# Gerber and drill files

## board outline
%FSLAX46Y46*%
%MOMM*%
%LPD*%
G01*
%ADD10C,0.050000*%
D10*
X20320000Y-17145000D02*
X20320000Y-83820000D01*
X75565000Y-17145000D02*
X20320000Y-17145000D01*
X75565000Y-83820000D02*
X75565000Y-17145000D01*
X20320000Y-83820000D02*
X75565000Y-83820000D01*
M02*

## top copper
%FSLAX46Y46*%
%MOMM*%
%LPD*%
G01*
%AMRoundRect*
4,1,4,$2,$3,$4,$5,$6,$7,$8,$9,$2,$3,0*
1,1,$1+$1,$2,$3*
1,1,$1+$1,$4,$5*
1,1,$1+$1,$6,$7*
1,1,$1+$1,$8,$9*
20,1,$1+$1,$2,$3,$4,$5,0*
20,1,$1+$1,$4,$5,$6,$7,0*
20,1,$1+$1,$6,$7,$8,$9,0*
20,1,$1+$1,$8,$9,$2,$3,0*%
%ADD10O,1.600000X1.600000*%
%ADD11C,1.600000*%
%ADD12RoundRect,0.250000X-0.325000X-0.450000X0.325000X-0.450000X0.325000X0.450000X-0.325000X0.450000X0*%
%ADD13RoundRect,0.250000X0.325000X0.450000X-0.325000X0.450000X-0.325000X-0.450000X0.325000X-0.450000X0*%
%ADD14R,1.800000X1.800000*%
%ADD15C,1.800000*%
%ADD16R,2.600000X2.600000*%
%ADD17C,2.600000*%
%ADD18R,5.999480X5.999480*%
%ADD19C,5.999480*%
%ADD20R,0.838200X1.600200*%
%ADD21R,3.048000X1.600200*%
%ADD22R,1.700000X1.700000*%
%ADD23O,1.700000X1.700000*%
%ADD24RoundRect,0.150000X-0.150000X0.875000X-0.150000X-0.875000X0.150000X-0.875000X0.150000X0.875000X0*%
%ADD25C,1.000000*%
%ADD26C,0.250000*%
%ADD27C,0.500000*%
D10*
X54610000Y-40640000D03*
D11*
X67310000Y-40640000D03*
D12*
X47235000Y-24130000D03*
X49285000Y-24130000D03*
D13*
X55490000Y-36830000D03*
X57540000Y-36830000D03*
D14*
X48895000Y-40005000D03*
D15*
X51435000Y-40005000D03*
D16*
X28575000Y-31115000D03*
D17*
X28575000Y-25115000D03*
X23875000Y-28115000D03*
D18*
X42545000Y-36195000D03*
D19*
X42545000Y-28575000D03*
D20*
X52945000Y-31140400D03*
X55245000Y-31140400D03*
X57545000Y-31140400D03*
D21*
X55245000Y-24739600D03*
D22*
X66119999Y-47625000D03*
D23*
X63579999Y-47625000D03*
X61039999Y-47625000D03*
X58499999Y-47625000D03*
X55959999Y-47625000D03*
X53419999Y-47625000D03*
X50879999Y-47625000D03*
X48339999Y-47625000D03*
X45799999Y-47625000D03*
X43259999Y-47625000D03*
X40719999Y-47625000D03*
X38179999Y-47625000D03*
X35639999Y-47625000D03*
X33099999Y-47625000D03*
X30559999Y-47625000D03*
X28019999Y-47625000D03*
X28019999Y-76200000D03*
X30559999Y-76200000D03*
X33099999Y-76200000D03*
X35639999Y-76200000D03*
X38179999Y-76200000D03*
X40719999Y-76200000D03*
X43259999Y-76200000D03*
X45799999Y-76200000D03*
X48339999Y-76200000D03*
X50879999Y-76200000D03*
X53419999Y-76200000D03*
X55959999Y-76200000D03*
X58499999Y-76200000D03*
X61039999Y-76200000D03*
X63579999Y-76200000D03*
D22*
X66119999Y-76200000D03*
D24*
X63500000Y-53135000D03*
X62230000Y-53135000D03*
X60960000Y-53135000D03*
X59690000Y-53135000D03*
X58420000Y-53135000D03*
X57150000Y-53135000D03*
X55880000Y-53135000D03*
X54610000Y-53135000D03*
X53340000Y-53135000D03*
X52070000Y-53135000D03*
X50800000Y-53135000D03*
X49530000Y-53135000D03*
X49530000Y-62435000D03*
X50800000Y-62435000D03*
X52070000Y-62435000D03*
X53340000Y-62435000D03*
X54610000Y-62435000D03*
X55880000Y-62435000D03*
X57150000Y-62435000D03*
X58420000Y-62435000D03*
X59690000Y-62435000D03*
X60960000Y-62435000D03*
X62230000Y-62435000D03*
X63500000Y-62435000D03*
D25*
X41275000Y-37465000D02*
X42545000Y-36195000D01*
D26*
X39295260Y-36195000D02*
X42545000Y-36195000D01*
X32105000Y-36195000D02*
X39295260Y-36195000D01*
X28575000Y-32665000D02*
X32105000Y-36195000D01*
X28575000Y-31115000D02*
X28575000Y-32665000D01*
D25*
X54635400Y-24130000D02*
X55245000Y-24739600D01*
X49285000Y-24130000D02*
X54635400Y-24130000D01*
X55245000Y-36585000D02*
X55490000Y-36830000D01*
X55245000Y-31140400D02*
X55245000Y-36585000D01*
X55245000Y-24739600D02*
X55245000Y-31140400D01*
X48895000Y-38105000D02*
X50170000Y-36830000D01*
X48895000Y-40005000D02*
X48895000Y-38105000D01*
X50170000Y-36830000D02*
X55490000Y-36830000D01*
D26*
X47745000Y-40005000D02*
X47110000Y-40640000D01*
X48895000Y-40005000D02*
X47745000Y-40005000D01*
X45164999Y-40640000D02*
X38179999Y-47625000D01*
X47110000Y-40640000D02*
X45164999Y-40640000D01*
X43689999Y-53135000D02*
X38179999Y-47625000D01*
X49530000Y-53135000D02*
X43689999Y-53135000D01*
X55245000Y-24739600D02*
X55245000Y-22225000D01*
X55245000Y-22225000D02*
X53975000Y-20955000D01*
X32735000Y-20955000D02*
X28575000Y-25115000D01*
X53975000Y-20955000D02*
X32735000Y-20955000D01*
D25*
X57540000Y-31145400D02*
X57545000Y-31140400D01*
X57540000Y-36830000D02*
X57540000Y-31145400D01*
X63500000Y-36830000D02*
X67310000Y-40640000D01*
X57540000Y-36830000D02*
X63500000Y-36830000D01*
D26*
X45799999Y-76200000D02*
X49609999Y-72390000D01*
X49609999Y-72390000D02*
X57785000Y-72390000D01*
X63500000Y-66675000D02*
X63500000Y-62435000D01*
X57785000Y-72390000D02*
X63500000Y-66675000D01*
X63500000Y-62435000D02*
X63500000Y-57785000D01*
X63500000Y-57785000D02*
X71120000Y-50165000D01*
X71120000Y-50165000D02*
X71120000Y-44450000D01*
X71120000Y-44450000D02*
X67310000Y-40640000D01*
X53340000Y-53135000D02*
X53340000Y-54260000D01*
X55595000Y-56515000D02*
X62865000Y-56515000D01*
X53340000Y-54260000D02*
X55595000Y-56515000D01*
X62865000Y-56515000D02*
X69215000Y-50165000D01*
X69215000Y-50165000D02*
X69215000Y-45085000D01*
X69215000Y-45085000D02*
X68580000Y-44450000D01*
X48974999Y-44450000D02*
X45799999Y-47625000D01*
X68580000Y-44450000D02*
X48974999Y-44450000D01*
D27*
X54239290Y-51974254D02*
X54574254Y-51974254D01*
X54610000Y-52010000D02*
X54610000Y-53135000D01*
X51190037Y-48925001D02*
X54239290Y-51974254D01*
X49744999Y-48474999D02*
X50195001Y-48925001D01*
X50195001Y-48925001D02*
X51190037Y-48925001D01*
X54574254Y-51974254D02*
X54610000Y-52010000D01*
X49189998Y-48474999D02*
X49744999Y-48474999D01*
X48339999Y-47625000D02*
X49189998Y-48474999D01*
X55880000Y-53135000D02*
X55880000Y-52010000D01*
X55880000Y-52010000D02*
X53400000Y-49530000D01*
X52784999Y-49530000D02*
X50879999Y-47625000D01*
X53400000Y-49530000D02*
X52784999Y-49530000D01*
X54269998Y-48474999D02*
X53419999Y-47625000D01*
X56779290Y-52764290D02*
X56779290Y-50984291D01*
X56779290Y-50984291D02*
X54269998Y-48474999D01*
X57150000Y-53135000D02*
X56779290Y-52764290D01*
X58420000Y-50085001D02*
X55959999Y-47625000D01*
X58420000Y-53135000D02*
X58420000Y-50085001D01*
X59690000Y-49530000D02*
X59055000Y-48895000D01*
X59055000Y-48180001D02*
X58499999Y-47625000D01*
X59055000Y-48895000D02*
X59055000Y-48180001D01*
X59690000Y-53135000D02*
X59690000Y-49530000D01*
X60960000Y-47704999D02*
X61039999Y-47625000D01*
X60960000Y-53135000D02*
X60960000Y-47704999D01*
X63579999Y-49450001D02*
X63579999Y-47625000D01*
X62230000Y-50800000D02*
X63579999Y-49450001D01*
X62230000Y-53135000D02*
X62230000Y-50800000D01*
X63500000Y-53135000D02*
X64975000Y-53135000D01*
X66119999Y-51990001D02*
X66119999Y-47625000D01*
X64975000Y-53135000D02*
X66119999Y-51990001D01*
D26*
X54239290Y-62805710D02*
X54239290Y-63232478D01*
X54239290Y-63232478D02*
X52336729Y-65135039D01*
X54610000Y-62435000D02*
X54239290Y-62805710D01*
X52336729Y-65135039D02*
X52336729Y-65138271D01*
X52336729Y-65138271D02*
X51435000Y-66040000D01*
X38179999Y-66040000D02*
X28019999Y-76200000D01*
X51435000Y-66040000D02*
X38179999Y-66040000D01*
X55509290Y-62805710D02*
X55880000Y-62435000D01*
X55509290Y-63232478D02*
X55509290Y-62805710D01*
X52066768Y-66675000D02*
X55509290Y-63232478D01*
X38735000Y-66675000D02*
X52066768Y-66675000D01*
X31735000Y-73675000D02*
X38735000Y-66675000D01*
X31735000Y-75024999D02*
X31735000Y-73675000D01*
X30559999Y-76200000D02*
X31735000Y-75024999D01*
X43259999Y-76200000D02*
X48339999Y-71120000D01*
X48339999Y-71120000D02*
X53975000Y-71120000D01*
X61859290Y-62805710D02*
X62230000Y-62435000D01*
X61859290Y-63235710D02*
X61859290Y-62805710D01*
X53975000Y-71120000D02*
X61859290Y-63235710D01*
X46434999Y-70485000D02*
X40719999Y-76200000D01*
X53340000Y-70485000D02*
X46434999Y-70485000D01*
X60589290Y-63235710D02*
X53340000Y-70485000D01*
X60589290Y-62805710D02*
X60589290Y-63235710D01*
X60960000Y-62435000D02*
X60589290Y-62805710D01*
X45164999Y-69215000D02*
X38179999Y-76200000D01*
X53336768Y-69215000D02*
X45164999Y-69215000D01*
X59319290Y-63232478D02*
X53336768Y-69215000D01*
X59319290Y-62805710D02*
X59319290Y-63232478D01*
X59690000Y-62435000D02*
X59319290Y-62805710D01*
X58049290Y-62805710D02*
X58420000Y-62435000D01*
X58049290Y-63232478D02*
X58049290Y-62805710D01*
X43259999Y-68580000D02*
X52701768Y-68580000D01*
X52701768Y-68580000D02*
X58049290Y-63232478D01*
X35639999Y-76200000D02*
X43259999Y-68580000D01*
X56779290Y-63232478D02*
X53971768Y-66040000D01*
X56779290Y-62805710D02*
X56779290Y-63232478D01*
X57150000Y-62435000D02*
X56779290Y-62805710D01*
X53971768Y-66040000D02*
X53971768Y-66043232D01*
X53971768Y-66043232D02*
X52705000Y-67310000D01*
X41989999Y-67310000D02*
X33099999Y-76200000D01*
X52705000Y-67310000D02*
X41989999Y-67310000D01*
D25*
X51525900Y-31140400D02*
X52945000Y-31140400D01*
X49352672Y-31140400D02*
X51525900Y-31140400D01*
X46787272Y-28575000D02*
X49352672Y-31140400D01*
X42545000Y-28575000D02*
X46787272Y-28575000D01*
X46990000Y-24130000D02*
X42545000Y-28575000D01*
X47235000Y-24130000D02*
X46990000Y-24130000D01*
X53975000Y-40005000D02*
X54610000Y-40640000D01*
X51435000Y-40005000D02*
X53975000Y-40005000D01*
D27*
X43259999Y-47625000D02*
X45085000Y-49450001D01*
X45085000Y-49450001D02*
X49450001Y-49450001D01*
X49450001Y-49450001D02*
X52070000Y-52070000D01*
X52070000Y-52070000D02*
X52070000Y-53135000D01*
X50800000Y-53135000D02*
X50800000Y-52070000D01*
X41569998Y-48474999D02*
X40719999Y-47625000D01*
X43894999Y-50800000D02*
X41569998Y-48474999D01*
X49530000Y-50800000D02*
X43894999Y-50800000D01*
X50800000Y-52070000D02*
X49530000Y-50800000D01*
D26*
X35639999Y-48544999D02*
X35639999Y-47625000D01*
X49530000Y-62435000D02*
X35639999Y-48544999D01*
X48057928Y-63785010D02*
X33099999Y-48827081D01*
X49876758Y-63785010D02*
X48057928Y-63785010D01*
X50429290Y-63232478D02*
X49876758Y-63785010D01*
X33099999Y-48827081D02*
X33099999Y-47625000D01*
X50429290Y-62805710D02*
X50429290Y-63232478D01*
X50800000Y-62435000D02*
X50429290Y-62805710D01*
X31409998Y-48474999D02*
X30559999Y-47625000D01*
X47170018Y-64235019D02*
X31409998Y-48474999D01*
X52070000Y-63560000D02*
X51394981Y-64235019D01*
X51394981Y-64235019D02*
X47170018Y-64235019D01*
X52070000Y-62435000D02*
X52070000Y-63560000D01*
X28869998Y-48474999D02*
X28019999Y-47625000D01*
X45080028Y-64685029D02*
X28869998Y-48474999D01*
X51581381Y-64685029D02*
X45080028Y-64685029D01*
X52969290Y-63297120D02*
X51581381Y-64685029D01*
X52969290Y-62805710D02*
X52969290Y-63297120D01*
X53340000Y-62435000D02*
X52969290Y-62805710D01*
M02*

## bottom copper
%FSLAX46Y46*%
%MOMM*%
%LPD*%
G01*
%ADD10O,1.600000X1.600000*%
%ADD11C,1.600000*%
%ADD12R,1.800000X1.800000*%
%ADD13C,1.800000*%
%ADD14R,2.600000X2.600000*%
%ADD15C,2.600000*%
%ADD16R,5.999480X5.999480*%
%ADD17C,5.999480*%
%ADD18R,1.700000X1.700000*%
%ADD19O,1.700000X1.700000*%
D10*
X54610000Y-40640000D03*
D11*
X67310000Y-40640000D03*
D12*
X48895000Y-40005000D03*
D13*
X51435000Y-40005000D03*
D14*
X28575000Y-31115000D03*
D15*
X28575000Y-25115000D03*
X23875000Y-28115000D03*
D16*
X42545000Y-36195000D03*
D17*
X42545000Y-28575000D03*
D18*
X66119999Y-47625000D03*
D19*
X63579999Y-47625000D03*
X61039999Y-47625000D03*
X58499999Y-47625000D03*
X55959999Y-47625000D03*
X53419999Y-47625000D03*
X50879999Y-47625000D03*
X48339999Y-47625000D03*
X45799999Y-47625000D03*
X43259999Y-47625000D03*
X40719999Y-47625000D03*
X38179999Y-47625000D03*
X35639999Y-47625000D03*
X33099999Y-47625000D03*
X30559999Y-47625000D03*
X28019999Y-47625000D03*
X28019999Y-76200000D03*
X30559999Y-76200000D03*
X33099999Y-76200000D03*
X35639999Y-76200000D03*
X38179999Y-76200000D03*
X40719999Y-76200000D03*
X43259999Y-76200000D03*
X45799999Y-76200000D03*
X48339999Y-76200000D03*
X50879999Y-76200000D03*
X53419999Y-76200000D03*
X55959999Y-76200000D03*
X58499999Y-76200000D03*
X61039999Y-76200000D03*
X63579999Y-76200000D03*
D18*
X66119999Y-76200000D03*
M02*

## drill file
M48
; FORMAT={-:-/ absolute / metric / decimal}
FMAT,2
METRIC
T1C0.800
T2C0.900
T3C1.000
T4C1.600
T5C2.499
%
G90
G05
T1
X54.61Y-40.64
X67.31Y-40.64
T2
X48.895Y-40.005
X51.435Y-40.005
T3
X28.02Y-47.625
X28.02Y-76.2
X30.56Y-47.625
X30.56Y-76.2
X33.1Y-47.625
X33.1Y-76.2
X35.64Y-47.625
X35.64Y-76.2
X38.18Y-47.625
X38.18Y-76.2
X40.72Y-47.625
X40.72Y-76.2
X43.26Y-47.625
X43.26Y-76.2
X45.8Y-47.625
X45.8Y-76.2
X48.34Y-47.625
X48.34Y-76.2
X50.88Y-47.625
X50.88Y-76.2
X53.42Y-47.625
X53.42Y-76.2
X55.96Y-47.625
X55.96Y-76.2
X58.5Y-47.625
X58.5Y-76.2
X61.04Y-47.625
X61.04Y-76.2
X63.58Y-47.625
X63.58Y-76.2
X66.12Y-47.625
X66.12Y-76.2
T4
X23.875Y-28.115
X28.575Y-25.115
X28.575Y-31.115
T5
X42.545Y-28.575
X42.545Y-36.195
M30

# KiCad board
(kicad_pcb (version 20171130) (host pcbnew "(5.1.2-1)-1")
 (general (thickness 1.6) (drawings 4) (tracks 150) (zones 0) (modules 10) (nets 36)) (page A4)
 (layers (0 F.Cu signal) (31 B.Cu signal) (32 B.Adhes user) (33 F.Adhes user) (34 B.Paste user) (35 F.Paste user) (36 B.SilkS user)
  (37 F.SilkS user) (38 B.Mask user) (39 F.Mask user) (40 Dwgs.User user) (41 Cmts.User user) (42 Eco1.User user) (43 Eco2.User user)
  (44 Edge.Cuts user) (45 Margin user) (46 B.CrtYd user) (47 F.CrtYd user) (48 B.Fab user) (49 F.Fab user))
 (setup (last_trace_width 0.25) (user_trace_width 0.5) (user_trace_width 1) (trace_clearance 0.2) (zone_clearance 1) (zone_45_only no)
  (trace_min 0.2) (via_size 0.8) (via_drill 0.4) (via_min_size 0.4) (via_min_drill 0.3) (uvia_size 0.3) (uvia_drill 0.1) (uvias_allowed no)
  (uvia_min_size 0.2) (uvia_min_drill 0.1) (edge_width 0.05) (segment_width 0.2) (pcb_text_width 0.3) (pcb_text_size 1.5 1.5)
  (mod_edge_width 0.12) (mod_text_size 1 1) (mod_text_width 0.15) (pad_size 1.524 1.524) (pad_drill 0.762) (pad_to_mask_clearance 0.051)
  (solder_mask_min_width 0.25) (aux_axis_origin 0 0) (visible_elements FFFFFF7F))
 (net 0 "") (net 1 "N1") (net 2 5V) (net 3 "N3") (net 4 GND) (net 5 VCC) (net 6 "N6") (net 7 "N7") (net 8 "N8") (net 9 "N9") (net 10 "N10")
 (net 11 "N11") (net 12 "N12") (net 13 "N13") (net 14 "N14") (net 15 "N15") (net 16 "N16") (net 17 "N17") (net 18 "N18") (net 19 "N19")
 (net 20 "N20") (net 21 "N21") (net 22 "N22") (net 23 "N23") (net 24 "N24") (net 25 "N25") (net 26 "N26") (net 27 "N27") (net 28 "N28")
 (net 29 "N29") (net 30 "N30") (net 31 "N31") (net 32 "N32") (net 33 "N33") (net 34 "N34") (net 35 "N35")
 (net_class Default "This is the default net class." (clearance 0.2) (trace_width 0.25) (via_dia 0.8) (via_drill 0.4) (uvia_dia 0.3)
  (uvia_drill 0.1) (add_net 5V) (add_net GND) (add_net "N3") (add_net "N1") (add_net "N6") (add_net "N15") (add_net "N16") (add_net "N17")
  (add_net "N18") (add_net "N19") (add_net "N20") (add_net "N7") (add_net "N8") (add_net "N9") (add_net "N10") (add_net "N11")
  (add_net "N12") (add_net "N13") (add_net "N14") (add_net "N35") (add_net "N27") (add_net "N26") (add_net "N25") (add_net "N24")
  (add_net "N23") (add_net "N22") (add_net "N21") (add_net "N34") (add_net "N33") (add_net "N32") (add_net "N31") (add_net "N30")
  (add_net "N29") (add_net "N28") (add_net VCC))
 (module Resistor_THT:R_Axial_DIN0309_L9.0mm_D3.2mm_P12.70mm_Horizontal (layer F.Cu) (at 67.31 40.64 180)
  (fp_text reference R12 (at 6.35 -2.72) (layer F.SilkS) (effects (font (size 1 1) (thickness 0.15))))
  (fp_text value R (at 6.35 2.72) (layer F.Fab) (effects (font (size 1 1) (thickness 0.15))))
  (pad 2 thru_hole oval (at 12.7 0 180) (size 1.6 1.6) (drill 0.8) (layers *.Cu *.Mask) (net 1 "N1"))
  (pad 1 thru_hole circle (at 0 0 180) (size 1.6 1.6) (drill 0.8) (layers *.Cu *.Mask) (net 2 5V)))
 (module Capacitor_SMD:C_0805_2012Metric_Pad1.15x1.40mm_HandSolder (layer F.Cu) (at 48.26 24.13)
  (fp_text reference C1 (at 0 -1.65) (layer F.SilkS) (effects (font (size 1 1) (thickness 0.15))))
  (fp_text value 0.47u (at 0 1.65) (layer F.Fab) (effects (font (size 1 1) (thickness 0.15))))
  (pad 1 smd roundrect (at -1.025 0) (size 1.15 1.4) (layers F.Cu F.Paste F.Mask) (roundrect_rratio 0.217391) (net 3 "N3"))
  (pad 2 smd roundrect (at 1.025 0) (size 1.15 1.4) (layers F.Cu F.Paste F.Mask) (roundrect_rratio 0.217391) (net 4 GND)))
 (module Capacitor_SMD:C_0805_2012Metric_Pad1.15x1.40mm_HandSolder (layer F.Cu) (at 56.515 36.83 180)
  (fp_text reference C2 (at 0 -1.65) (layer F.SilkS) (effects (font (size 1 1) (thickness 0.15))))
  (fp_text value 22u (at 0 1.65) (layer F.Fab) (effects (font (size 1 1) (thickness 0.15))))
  (pad 2 smd roundrect (at 1.025 0 180) (size 1.15 1.4) (layers F.Cu F.Paste F.Mask) (roundrect_rratio 0.217391) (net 4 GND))
  (pad 1 smd roundrect (at -1.025 0 180) (size 1.15 1.4) (layers F.Cu F.Paste F.Mask) (roundrect_rratio 0.217391) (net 2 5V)))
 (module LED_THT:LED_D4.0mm (layer F.Cu) (at 48.895 40.005)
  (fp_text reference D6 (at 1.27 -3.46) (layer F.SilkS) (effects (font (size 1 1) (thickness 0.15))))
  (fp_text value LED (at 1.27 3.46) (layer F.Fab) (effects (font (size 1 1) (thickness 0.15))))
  (pad 1 thru_hole rect (at 0 0) (size 1.8 1.8) (drill 0.9) (layers *.Cu *.Mask) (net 4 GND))
  (pad 2 thru_hole circle (at 2.54 0) (size 1.8 1.8) (drill 0.9) (layers *.Cu *.Mask) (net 1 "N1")))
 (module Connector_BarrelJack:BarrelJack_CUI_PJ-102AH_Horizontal (layer F.Cu) (at 28.575 31.115 180)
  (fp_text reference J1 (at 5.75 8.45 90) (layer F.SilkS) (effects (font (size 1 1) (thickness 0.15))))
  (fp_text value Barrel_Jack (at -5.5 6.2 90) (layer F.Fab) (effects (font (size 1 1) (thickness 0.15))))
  (pad 1 thru_hole rect (at 0 0 180) (size 2.6 2.6) (drill 1.6) (layers *.Cu *.Mask) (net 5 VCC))
  (pad 2 thru_hole circle (at 0 6 180) (size 2.6 2.6) (drill 1.6) (layers *.Cu *.Mask) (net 4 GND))
  (pad 3 thru_hole circle (at 4.7 3 180) (size 2.6 2.6) (drill 1.6) (layers *.Cu *.Mask)))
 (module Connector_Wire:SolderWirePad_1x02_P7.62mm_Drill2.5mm (layer F.Cu) (at 42.545 36.195 90)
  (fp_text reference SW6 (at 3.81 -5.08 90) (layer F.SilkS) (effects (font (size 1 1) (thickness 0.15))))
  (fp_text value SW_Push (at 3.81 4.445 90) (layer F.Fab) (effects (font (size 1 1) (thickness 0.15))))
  (pad 1 thru_hole rect (at 0 0 90) (size 5.99948 5.99948) (drill 2.49936) (layers *.Cu *.Mask) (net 5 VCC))
  (pad 2 thru_hole circle (at 7.62 0 90) (size 5.99948 5.99948) (drill 2.49936) (layers *.Cu *.Mask) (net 3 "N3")))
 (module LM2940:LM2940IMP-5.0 (layer F.Cu) (at 55.245 27.94 90)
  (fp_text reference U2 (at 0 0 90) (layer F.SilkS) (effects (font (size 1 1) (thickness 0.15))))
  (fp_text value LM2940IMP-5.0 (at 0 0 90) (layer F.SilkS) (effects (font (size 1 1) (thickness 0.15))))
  (pad 1 smd rect (at -3.2004 -2.3 90) (size 1.6002 0.8382) (layers F.Cu F.Paste F.Mask) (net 3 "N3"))
  (pad 2 smd rect (at -3.2004 0 90) (size 1.6002 0.8382) (layers F.Cu F.Paste F.Mask) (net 4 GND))
  (pad 3 smd rect (at -3.2004 2.3 90) (size 1.6002 0.8382) (layers F.Cu F.Paste F.Mask) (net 2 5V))
  (pad 4 smd rect (at 3.2004 0 90) (size 1.6002 3.048) (layers F.Cu F.Paste F.Mask) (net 4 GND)))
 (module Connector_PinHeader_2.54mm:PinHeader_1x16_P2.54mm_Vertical (layer F.Cu) (at 66.119999 47.625 270)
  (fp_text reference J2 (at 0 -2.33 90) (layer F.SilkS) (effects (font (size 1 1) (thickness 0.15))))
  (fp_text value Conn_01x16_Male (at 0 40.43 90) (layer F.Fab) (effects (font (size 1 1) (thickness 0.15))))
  (pad 1 thru_hole rect (at 0 0 270) (size 1.7 1.7) (drill 1) (layers *.Cu *.Mask) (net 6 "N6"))
  (pad 2 thru_hole oval (at 0 2.54 270) (size 1.7 1.7) (drill 1) (layers *.Cu *.Mask) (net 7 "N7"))
  (pad 3 thru_hole oval (at 0 5.08 270) (size 1.7 1.7) (drill 1) (layers *.Cu *.Mask) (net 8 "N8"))
  (pad 4 thru_hole oval (at 0 7.62 270) (size 1.7 1.7) (drill 1) (layers *.Cu *.Mask) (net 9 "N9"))
  (pad 5 thru_hole oval (at 0 10.16 270) (size 1.7 1.7) (drill 1) (layers *.Cu *.Mask) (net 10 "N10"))
  (pad 6 thru_hole oval (at 0 12.7 270) (size 1.7 1.7) (drill 1) (layers *.Cu *.Mask) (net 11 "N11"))
  (pad 7 thru_hole oval (at 0 15.24 270) (size 1.7 1.7) (drill 1) (layers *.Cu *.Mask) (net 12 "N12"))
  (pad 8 thru_hole oval (at 0 17.78 270) (size 1.7 1.7) (drill 1) (layers *.Cu *.Mask) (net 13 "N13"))
  (pad 9 thru_hole oval (at 0 20.32 270) (size 1.7 1.7) (drill 1) (layers *.Cu *.Mask) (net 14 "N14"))
  (pad 10 thru_hole oval (at 0 22.86 270) (size 1.7 1.7) (drill 1) (layers *.Cu *.Mask) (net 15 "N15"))
  (pad 11 thru_hole oval (at 0 25.4 270) (size 1.7 1.7) (drill 1) (layers *.Cu *.Mask) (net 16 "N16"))
  (pad 12 thru_hole oval (at 0 27.94 270) (size 1.7 1.7) (drill 1) (layers *.Cu *.Mask) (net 4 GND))
  (pad 13 thru_hole oval (at 0 30.48 270) (size 1.7 1.7) (drill 1) (layers *.Cu *.Mask) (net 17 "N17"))
  (pad 14 thru_hole oval (at 0 33.02 270) (size 1.7 1.7) (drill 1) (layers *.Cu *.Mask) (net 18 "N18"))
  (pad 15 thru_hole oval (at 0 35.56 270) (size 1.7 1.7) (drill 1) (layers *.Cu *.Mask) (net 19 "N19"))
  (pad 16 thru_hole oval (at 0 38.1 270) (size 1.7 1.7) (drill 1) (layers *.Cu *.Mask) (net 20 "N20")))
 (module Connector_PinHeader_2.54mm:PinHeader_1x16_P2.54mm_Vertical (layer F.Cu) (at 66.119999 76.2 270)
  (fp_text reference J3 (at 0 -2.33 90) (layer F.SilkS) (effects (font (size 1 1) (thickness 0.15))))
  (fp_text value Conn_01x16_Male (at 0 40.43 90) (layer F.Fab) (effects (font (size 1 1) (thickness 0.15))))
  (pad 16 thru_hole oval (at 0 38.1 270) (size 1.7 1.7) (drill 1) (layers *.Cu *.Mask) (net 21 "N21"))
  (pad 15 thru_hole oval (at 0 35.56 270) (size 1.7 1.7) (drill 1) (layers *.Cu *.Mask) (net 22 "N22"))
  (pad 14 thru_hole oval (at 0 33.02 270) (size 1.7 1.7) (drill 1) (layers *.Cu *.Mask) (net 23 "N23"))
  (pad 13 thru_hole oval (at 0 30.48 270) (size 1.7 1.7) (drill 1) (layers *.Cu *.Mask) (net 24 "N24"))
  (pad 12 thru_hole oval (at 0 27.94 270) (size 1.7 1.7) (drill 1) (layers *.Cu *.Mask) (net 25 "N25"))
  (pad 11 thru_hole oval (at 0 25.4 270) (size 1.7 1.7) (drill 1) (layers *.Cu *.Mask) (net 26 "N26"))
  (pad 10 thru_hole oval (at 0 22.86 270) (size 1.7 1.7) (drill 1) (layers *.Cu *.Mask) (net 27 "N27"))
  (pad 9 thru_hole oval (at 0 20.32 270) (size 1.7 1.7) (drill 1) (layers *.Cu *.Mask) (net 2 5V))
  (pad 8 thru_hole oval (at 0 17.78 270) (size 1.7 1.7) (drill 1) (layers *.Cu *.Mask) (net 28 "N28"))
  (pad 7 thru_hole oval (at 0 15.24 270) (size 1.7 1.7) (drill 1) (layers *.Cu *.Mask) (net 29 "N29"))
  (pad 6 thru_hole oval (at 0 12.7 270) (size 1.7 1.7) (drill 1) (layers *.Cu *.Mask) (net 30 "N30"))
  (pad 5 thru_hole oval (at 0 10.16 270) (size 1.7 1.7) (drill 1) (layers *.Cu *.Mask) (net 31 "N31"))
  (pad 4 thru_hole oval (at 0 7.62 270) (size 1.7 1.7) (drill 1) (layers *.Cu *.Mask) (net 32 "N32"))
  (pad 3 thru_hole oval (at 0 5.08 270) (size 1.7 1.7) (drill 1) (layers *.Cu *.Mask) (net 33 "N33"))
  (pad 2 thru_hole oval (at 0 2.54 270) (size 1.7 1.7) (drill 1) (layers *.Cu *.Mask) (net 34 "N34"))
  (pad 1 thru_hole rect (at 0 0 270) (size 1.7 1.7) (drill 1) (layers *.Cu *.Mask) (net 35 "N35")))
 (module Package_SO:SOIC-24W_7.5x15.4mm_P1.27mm (layer F.Cu) (at 56.515 57.785 270)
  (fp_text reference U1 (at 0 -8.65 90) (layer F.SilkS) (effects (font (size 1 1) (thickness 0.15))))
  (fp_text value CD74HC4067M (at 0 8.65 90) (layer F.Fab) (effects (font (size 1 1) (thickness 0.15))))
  (pad 1 smd roundrect (at -4.65 -6.985 270) (size 2.05 0.6) (layers F.Cu F.Paste F.Mask) (roundrect_rratio 0.25) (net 6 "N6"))
  (pad 2 smd roundrect (at -4.65 -5.715 270) (size 2.05 0.6) (layers F.Cu F.Paste F.Mask) (roundrect_rratio 0.25) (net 7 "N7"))
  (pad 3 smd roundrect (at -4.65 -4.445 270) (size 2.05 0.6) (layers F.Cu F.Paste F.Mask) (roundrect_rratio 0.25) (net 8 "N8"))
  (pad 4 smd roundrect (at -4.65 -3.175 270) (size 2.05 0.6) (layers F.Cu F.Paste F.Mask) (roundrect_rratio 0.25) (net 9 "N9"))
  (pad 5 smd roundrect (at -4.65 -1.905 270) (size 2.05 0.6) (layers F.Cu F.Paste F.Mask) (roundrect_rratio 0.25) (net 10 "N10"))
  (pad 6 smd roundrect (at -4.65 -0.635 270) (size 2.05 0.6) (layers F.Cu F.Paste F.Mask) (roundrect_rratio 0.25) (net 11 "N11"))
  (pad 7 smd roundrect (at -4.65 0.635 270) (size 2.05 0.6) (layers F.Cu F.Paste F.Mask) (roundrect_rratio 0.25) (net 12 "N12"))
  (pad 8 smd roundrect (at -4.65 1.905 270) (size 2.05 0.6) (layers F.Cu F.Paste F.Mask) (roundrect_rratio 0.25) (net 13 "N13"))
  (pad 9 smd roundrect (at -4.65 3.175 270) (size 2.05 0.6) (layers F.Cu F.Paste F.Mask) (roundrect_rratio 0.25) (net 14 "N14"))
  (pad 10 smd roundrect (at -4.65 4.445 270) (size 2.05 0.6) (layers F.Cu F.Paste F.Mask) (roundrect_rratio 0.25) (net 15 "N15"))
  (pad 11 smd roundrect (at -4.65 5.715 270) (size 2.05 0.6) (layers F.Cu F.Paste F.Mask) (roundrect_rratio 0.25) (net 16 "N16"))
  (pad 12 smd roundrect (at -4.65 6.985 270) (size 2.05 0.6) (layers F.Cu F.Paste F.Mask) (roundrect_rratio 0.25) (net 4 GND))
  (pad 13 smd roundrect (at 4.65 6.985 270) (size 2.05 0.6) (layers F.Cu F.Paste F.Mask) (roundrect_rratio 0.25) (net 17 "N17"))
  (pad 14 smd roundrect (at 4.65 5.715 270) (size 2.05 0.6) (layers F.Cu F.Paste F.Mask) (roundrect_rratio 0.25) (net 18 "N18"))
  (pad 15 smd roundrect (at 4.65 4.445 270) (size 2.05 0.6) (layers F.Cu F.Paste F.Mask) (roundrect_rratio 0.25) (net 19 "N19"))
  (pad 16 smd roundrect (at 4.65 3.175 270) (size 2.05 0.6) (layers F.Cu F.Paste F.Mask) (roundrect_rratio 0.25) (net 20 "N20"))
  (pad 17 smd roundrect (at 4.65 1.905 270) (size 2.05 0.6) (layers F.Cu F.Paste F.Mask) (roundrect_rratio 0.25) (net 21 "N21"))
  (pad 18 smd roundrect (at 4.65 0.635 270) (size 2.05 0.6) (layers F.Cu F.Paste F.Mask) (roundrect_rratio 0.25) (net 22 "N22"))
  (pad 19 smd roundrect (at 4.65 -0.635 270) (size 2.05 0.6) (layers F.Cu F.Paste F.Mask) (roundrect_rratio 0.25) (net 23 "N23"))
  (pad 20 smd roundrect (at 4.65 -1.905 270) (size 2.05 0.6) (layers F.Cu F.Paste F.Mask) (roundrect_rratio 0.25) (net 24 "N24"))
  (pad 21 smd roundrect (at 4.65 -3.175 270) (size 2.05 0.6) (layers F.Cu F.Paste F.Mask) (roundrect_rratio 0.25) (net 25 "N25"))
  (pad 22 smd roundrect (at 4.65 -4.445 270) (size 2.05 0.6) (layers F.Cu F.Paste F.Mask) (roundrect_rratio 0.25) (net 26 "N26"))
  (pad 23 smd roundrect (at 4.65 -5.715 270) (size 2.05 0.6) (layers F.Cu F.Paste F.Mask) (roundrect_rratio 0.25) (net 27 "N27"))
  (pad 24 smd roundrect (at 4.65 -6.985 270) (size 2.05 0.6) (layers F.Cu F.Paste F.Mask) (roundrect_rratio 0.25) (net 2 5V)))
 (gr_line (start 20.32 17.145) (end 20.32 83.82) (layer Edge.Cuts) (width 0.05))
 (gr_line (start 75.565 17.145) (end 20.32 17.145) (layer Edge.Cuts) (width 0.05))
 (gr_line (start 75.565 83.82) (end 75.565 17.145) (layer Edge.Cuts) (width 0.05))
 (gr_line (start 20.32 83.82) (end 75.565 83.82) (layer Edge.Cuts) (width 0.05))
 (segment (start 41.275 37.465) (end 42.545 36.195) (width 1) (layer F.Cu) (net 5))
 (segment (start 39.29526 36.195) (end 42.545 36.195) (width 0.25) (layer F.Cu) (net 5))
 (segment (start 32.105 36.195) (end 39.29526 36.195) (width 0.25) (layer F.Cu) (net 5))
 (segment (start 28.575 32.665) (end 32.105 36.195) (width 0.25) (layer F.Cu) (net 5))
 (segment (start 28.575 31.115) (end 28.575 32.665) (width 0.25) (layer F.Cu) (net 5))
 (segment (start 54.6354 24.13) (end 55.245 24.7396) (width 1) (layer F.Cu) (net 4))
 (segment (start 49.285 24.13) (end 54.6354 24.13) (width 1) (layer F.Cu) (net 4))
 (segment (start 55.245 36.585) (end 55.49 36.83) (width 1) (layer F.Cu) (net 4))
 (segment (start 55.245 31.1404) (end 55.245 36.585) (width 1) (layer F.Cu) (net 4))
 (segment (start 55.245 24.7396) (end 55.245 31.1404) (width 1) (layer F.Cu) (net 4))
 (segment (start 48.895 38.105) (end 50.17 36.83) (width 1) (layer F.Cu) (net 4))
 (segment (start 48.895 40.005) (end 48.895 38.105) (width 1) (layer F.Cu) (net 4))
 (segment (start 50.17 36.83) (end 55.49 36.83) (width 1) (layer F.Cu) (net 4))
 (segment (start 47.745 40.005) (end 47.11 40.64) (width 0.25) (layer F.Cu) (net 4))
 (segment (start 48.895 40.005) (end 47.745 40.005) (width 0.25) (layer F.Cu) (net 4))
 (segment (start 45.164999 40.64) (end 38.179999 47.625) (width 0.25) (layer F.Cu) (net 4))
 (segment (start 47.11 40.64) (end 45.164999 40.64) (width 0.25) (layer F.Cu) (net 4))
 (segment (start 43.689999 53.135) (end 38.179999 47.625) (width 0.25) (layer F.Cu) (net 4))
 (segment (start 49.53 53.135) (end 43.689999 53.135) (width 0.25) (layer F.Cu) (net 4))
 (segment (start 55.245 24.7396) (end 55.245 22.225) (width 0.25) (layer F.Cu) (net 4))
 (segment (start 55.245 22.225) (end 53.975 20.955) (width 0.25) (layer F.Cu) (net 4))
 (segment (start 32.735 20.955) (end 28.575 25.115) (width 0.25) (layer F.Cu) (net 4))
 (segment (start 53.975 20.955) (end 32.735 20.955) (width 0.25) (layer F.Cu) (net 4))
 (segment (start 57.54 31.1454) (end 57.545 31.1404) (width 1) (layer F.Cu) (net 2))
 (segment (start 57.54 36.83) (end 57.54 31.1454) (width 1) (layer F.Cu) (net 2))
 (segment (start 63.5 36.83) (end 67.31 40.64) (width 1) (layer F.Cu) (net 2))
 (segment (start 57.54 36.83) (end 63.5 36.83) (width 1) (layer F.Cu) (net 2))
 (segment (start 45.799999 76.2) (end 49.609999 72.39) (width 0.25) (layer F.Cu) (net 2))
 (segment (start 49.609999 72.39) (end 57.785 72.39) (width 0.25) (layer F.Cu) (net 2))
 (segment (start 63.5 66.675) (end 63.5 62.435) (width 0.25) (layer F.Cu) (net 2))
 (segment (start 57.785 72.39) (end 63.5 66.675) (width 0.25) (layer F.Cu) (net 2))
 (segment (start 63.5 62.435) (end 63.5 57.785) (width 0.25) (layer F.Cu) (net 2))
 (segment (start 63.5 57.785) (end 71.12 50.165) (width 0.25) (layer F.Cu) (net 2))
 (segment (start 71.12 50.165) (end 71.12 44.45) (width 0.25) (layer F.Cu) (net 2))
 (segment (start 71.12 44.45) (end 67.31 40.64) (width 0.25) (layer F.Cu) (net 2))
 (segment (start 53.34 53.135) (end 53.34 54.26) (width 0.25) (layer F.Cu) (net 14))
 (segment (start 55.595 56.515) (end 62.865 56.515) (width 0.25) (layer F.Cu) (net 14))
 (segment (start 53.34 54.26) (end 55.595 56.515) (width 0.25) (layer F.Cu) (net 14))
 (segment (start 62.865 56.515) (end 69.215 50.165) (width 0.25) (layer F.Cu) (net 14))
 (segment (start 69.215 50.165) (end 69.215 45.085) (width 0.25) (layer F.Cu) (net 14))
 (segment (start 69.215 45.085) (end 68.58 44.45) (width 0.25) (layer F.Cu) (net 14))
 (segment (start 48.974999 44.45) (end 45.799999 47.625) (width 0.25) (layer F.Cu) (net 14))
 (segment (start 68.58 44.45) (end 48.974999 44.45) (width 0.25) (layer F.Cu) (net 14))
 (segment (start 54.23929 51.974254) (end 54.574254 51.974254) (width 0.5) (layer F.Cu) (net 13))
 (segment (start 54.61 52.01) (end 54.61 53.135) (width 0.5) (layer F.Cu) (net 13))
 (segment (start 51.190037 48.925001) (end 54.23929 51.974254) (width 0.5) (layer F.Cu) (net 13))
 (segment (start 49.744999 48.474999) (end 50.195001 48.925001) (width 0.5) (layer F.Cu) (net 13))
 (segment (start 50.195001 48.925001) (end 51.190037 48.925001) (width 0.5) (layer F.Cu) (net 13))
 (segment (start 54.574254 51.974254) (end 54.61 52.01) (width 0.5) (layer F.Cu) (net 13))
 (segment (start 49.189998 48.474999) (end 49.744999 48.474999) (width 0.5) (layer F.Cu) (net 13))
 (segment (start 48.339999 47.625) (end 49.189998 48.474999) (width 0.5) (layer F.Cu) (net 13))
 (segment (start 55.88 53.135) (end 55.88 52.01) (width 0.5) (layer F.Cu) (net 12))
 (segment (start 55.88 52.01) (end 53.4 49.53) (width 0.5) (layer F.Cu) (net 12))
 (segment (start 52.784999 49.53) (end 50.879999 47.625) (width 0.5) (layer F.Cu) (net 12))
 (segment (start 53.4 49.53) (end 52.784999 49.53) (width 0.5) (layer F.Cu) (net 12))
 (segment (start 54.269998 48.474999) (end 53.419999 47.625) (width 0.5) (layer F.Cu) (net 11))
 (segment (start 56.77929 52.76429) (end 56.77929 50.984291) (width 0.5) (layer F.Cu) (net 11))
 (segment (start 56.77929 50.984291) (end 54.269998 48.474999) (width 0.5) (layer F.Cu) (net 11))
 (segment (start 57.15 53.135) (end 56.77929 52.76429) (width 0.5) (layer F.Cu) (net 11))
 (segment (start 58.42 50.085001) (end 55.959999 47.625) (width 0.5) (layer F.Cu) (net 10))
 (segment (start 58.42 53.135) (end 58.42 50.085001) (width 0.5) (layer F.Cu) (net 10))
 (segment (start 59.69 49.53) (end 59.055 48.895) (width 0.5) (layer F.Cu) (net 9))
 (segment (start 59.055 48.180001) (end 58.499999 47.625) (width 0.5) (layer F.Cu) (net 9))
 (segment (start 59.055 48.895) (end 59.055 48.180001) (width 0.5) (layer F.Cu) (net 9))
 (segment (start 59.69 53.135) (end 59.69 49.53) (width 0.5) (layer F.Cu) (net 9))
 (segment (start 60.96 47.704999) (end 61.039999 47.625) (width 0.5) (layer F.Cu) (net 8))
 (segment (start 60.96 53.135) (end 60.96 47.704999) (width 0.5) (layer F.Cu) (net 8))
 (segment (start 63.579999 49.450001) (end 63.579999 47.625) (width 0.5) (layer F.Cu) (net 7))
 (segment (start 62.23 50.8) (end 63.579999 49.450001) (width 0.5) (layer F.Cu) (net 7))
 (segment (start 62.23 53.135) (end 62.23 50.8) (width 0.5) (layer F.Cu) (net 7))
 (segment (start 63.5 53.135) (end 64.975 53.135) (width 0.5) (layer F.Cu) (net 6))
 (segment (start 66.119999 51.990001) (end 66.119999 47.625) (width 0.5) (layer F.Cu) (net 6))
 (segment (start 64.975 53.135) (end 66.119999 51.990001) (width 0.5) (layer F.Cu) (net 6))
 (segment (start 54.23929 62.80571) (end 54.23929 63.232478) (width 0.25) (layer F.Cu) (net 21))
 (segment (start 54.23929 63.232478) (end 52.336729 65.135039) (width 0.25) (layer F.Cu) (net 21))
 (segment (start 54.61 62.435) (end 54.23929 62.80571) (width 0.25) (layer F.Cu) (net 21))
 (segment (start 52.336729 65.135039) (end 52.336729 65.138271) (width 0.25) (layer F.Cu) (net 21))
 (segment (start 52.336729 65.138271) (end 51.435 66.04) (width 0.25) (layer F.Cu) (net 21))
 (segment (start 38.179999 66.04) (end 28.019999 76.2) (width 0.25) (layer F.Cu) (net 21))
 (segment (start 51.435 66.04) (end 38.179999 66.04) (width 0.25) (layer F.Cu) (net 21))
 (segment (start 55.50929 62.80571) (end 55.88 62.435) (width 0.25) (layer F.Cu) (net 22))
 (segment (start 55.50929 63.232478) (end 55.50929 62.80571) (width 0.25) (layer F.Cu) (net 22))
 (segment (start 52.066768 66.675) (end 55.50929 63.232478) (width 0.25) (layer F.Cu) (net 22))
 (segment (start 38.735 66.675) (end 52.066768 66.675) (width 0.25) (layer F.Cu) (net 22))
 (segment (start 31.735 73.675) (end 38.735 66.675) (width 0.25) (layer F.Cu) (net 22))
 (segment (start 31.735 75.024999) (end 31.735 73.675) (width 0.25) (layer F.Cu) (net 22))
 (segment (start 30.559999 76.2) (end 31.735 75.024999) (width 0.25) (layer F.Cu) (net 22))
 (segment (start 43.259999 76.2) (end 48.339999 71.12) (width 0.25) (layer F.Cu) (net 27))
 (segment (start 48.339999 71.12) (end 53.975 71.12) (width 0.25) (layer F.Cu) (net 27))
 (segment (start 61.85929 62.80571) (end 62.23 62.435) (width 0.25) (layer F.Cu) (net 27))
 (segment (start 61.85929 63.23571) (end 61.85929 62.80571) (width 0.25) (layer F.Cu) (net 27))
 (segment (start 53.975 71.12) (end 61.85929 63.23571) (width 0.25) (layer F.Cu) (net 27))
 (segment (start 46.434999 70.485) (end 40.719999 76.2) (width 0.25) (layer F.Cu) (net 26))
 (segment (start 53.34 70.485) (end 46.434999 70.485) (width 0.25) (layer F.Cu) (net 26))
 (segment (start 60.58929 63.23571) (end 53.34 70.485) (width 0.25) (layer F.Cu) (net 26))
 (segment (start 60.58929 62.80571) (end 60.58929 63.23571) (width 0.25) (layer F.Cu) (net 26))
 (segment (start 60.96 62.435) (end 60.58929 62.80571) (width 0.25) (layer F.Cu) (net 26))
 (segment (start 45.164999 69.215) (end 38.179999 76.2) (width 0.25) (layer F.Cu) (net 25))
 (segment (start 53.336768 69.215) (end 45.164999 69.215) (width 0.25) (layer F.Cu) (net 25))
 (segment (start 59.31929 63.232478) (end 53.336768 69.215) (width 0.25) (layer F.Cu) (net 25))
 (segment (start 59.31929 62.80571) (end 59.31929 63.232478) (width 0.25) (layer F.Cu) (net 25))
 (segment (start 59.69 62.435) (end 59.31929 62.80571) (width 0.25) (layer F.Cu) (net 25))
 (segment (start 58.04929 62.80571) (end 58.42 62.435) (width 0.25) (layer F.Cu) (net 24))
 (segment (start 58.04929 63.232478) (end 58.04929 62.80571) (width 0.25) (layer F.Cu) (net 24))
 (segment (start 43.259999 68.58) (end 52.701768 68.58) (width 0.25) (layer F.Cu) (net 24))
 (segment (start 52.701768 68.58) (end 58.04929 63.232478) (width 0.25) (layer F.Cu) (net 24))
 (segment (start 35.639999 76.2) (end 43.259999 68.58) (width 0.25) (layer F.Cu) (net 24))
 (segment (start 56.77929 63.232478) (end 53.971768 66.04) (width 0.25) (layer F.Cu) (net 23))
 (segment (start 56.77929 62.80571) (end 56.77929 63.232478) (width 0.25) (layer F.Cu) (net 23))
 (segment (start 57.15 62.435) (end 56.77929 62.80571) (width 0.25) (layer F.Cu) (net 23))
 (segment (start 53.971768 66.04) (end 53.971768 66.043232) (width 0.25) (layer F.Cu) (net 23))
 (segment (start 53.971768 66.043232) (end 52.705 67.31) (width 0.25) (layer F.Cu) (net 23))
 (segment (start 41.989999 67.31) (end 33.099999 76.2) (width 0.25) (layer F.Cu) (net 23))
 (segment (start 52.705 67.31) (end 41.989999 67.31) (width 0.25) (layer F.Cu) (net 23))
 (segment (start 51.5259 31.1404) (end 52.945 31.1404) (width 1) (layer F.Cu) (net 3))
 (segment (start 49.352672 31.1404) (end 51.5259 31.1404) (width 1) (layer F.Cu) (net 3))
 (segment (start 46.787272 28.575) (end 49.352672 31.1404) (width 1) (layer F.Cu) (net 3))
 (segment (start 42.545 28.575) (end 46.787272 28.575) (width 1) (layer F.Cu) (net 3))
 (segment (start 46.99 24.13) (end 42.545 28.575) (width 1) (layer F.Cu) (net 3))
 (segment (start 47.235 24.13) (end 46.99 24.13) (width 1) (layer F.Cu) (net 3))
 (segment (start 53.975 40.005) (end 54.61 40.64) (width 1) (layer F.Cu) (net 1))
 (segment (start 51.435 40.005) (end 53.975 40.005) (width 1) (layer F.Cu) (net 1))
 (segment (start 43.259999 47.625) (end 45.085 49.450001) (width 0.5) (layer F.Cu) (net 15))
 (segment (start 45.085 49.450001) (end 49.450001 49.450001) (width 0.5) (layer F.Cu) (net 15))
 (segment (start 49.450001 49.450001) (end 52.07 52.07) (width 0.5) (layer F.Cu) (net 15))
 (segment (start 52.07 52.07) (end 52.07 53.135) (width 0.5) (layer F.Cu) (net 15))
 (segment (start 50.8 53.135) (end 50.8 52.07) (width 0.5) (layer F.Cu) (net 16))
 (segment (start 41.569998 48.474999) (end 40.719999 47.625) (width 0.5) (layer F.Cu) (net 16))
 (segment (start 43.894999 50.8) (end 41.569998 48.474999) (width 0.5) (layer F.Cu) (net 16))
 (segment (start 49.53 50.8) (end 43.894999 50.8) (width 0.5) (layer F.Cu) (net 16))
 (segment (start 50.8 52.07) (end 49.53 50.8) (width 0.5) (layer F.Cu) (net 16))
 (segment (start 35.639999 48.544999) (end 35.639999 47.625) (width 0.25) (layer F.Cu) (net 17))
 (segment (start 49.53 62.435) (end 35.639999 48.544999) (width 0.25) (layer F.Cu) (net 17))
 (segment (start 48.057928 63.78501) (end 33.099999 48.827081) (width 0.25) (layer F.Cu) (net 18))
 (segment (start 49.876758 63.78501) (end 48.057928 63.78501) (width 0.25) (layer F.Cu) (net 18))
 (segment (start 50.42929 63.232478) (end 49.876758 63.78501) (width 0.25) (layer F.Cu) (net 18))
 (segment (start 33.099999 48.827081) (end 33.099999 47.625) (width 0.25) (layer F.Cu) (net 18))
 (segment (start 50.42929 62.80571) (end 50.42929 63.232478) (width 0.25) (layer F.Cu) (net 18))
 (segment (start 50.8 62.435) (end 50.42929 62.80571) (width 0.25) (layer F.Cu) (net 18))
 (segment (start 31.409998 48.474999) (end 30.559999 47.625) (width 0.25) (layer F.Cu) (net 19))
 (segment (start 47.170018 64.235019) (end 31.409998 48.474999) (width 0.25) (layer F.Cu) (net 19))
 (segment (start 52.07 63.56) (end 51.394981 64.235019) (width 0.25) (layer F.Cu) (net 19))
 (segment (start 51.394981 64.235019) (end 47.170018 64.235019) (width 0.25) (layer F.Cu) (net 19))
 (segment (start 52.07 62.435) (end 52.07 63.56) (width 0.25) (layer F.Cu) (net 19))
 (segment (start 28.869998 48.474999) (end 28.019999 47.625) (width 0.25) (layer F.Cu) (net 20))
 (segment (start 45.080028 64.685029) (end 28.869998 48.474999) (width 0.25) (layer F.Cu) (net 20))
 (segment (start 51.581381 64.685029) (end 45.080028 64.685029) (width 0.25) (layer F.Cu) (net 20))
 (segment (start 52.96929 63.29712) (end 51.581381 64.685029) (width 0.25) (layer F.Cu) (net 20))
 (segment (start 52.96929 62.80571) (end 52.96929 63.29712) (width 0.25) (layer F.Cu) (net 20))
 (segment (start 53.34 62.435) (end 52.96929 62.80571) (width 0.25) (layer F.Cu) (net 20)))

